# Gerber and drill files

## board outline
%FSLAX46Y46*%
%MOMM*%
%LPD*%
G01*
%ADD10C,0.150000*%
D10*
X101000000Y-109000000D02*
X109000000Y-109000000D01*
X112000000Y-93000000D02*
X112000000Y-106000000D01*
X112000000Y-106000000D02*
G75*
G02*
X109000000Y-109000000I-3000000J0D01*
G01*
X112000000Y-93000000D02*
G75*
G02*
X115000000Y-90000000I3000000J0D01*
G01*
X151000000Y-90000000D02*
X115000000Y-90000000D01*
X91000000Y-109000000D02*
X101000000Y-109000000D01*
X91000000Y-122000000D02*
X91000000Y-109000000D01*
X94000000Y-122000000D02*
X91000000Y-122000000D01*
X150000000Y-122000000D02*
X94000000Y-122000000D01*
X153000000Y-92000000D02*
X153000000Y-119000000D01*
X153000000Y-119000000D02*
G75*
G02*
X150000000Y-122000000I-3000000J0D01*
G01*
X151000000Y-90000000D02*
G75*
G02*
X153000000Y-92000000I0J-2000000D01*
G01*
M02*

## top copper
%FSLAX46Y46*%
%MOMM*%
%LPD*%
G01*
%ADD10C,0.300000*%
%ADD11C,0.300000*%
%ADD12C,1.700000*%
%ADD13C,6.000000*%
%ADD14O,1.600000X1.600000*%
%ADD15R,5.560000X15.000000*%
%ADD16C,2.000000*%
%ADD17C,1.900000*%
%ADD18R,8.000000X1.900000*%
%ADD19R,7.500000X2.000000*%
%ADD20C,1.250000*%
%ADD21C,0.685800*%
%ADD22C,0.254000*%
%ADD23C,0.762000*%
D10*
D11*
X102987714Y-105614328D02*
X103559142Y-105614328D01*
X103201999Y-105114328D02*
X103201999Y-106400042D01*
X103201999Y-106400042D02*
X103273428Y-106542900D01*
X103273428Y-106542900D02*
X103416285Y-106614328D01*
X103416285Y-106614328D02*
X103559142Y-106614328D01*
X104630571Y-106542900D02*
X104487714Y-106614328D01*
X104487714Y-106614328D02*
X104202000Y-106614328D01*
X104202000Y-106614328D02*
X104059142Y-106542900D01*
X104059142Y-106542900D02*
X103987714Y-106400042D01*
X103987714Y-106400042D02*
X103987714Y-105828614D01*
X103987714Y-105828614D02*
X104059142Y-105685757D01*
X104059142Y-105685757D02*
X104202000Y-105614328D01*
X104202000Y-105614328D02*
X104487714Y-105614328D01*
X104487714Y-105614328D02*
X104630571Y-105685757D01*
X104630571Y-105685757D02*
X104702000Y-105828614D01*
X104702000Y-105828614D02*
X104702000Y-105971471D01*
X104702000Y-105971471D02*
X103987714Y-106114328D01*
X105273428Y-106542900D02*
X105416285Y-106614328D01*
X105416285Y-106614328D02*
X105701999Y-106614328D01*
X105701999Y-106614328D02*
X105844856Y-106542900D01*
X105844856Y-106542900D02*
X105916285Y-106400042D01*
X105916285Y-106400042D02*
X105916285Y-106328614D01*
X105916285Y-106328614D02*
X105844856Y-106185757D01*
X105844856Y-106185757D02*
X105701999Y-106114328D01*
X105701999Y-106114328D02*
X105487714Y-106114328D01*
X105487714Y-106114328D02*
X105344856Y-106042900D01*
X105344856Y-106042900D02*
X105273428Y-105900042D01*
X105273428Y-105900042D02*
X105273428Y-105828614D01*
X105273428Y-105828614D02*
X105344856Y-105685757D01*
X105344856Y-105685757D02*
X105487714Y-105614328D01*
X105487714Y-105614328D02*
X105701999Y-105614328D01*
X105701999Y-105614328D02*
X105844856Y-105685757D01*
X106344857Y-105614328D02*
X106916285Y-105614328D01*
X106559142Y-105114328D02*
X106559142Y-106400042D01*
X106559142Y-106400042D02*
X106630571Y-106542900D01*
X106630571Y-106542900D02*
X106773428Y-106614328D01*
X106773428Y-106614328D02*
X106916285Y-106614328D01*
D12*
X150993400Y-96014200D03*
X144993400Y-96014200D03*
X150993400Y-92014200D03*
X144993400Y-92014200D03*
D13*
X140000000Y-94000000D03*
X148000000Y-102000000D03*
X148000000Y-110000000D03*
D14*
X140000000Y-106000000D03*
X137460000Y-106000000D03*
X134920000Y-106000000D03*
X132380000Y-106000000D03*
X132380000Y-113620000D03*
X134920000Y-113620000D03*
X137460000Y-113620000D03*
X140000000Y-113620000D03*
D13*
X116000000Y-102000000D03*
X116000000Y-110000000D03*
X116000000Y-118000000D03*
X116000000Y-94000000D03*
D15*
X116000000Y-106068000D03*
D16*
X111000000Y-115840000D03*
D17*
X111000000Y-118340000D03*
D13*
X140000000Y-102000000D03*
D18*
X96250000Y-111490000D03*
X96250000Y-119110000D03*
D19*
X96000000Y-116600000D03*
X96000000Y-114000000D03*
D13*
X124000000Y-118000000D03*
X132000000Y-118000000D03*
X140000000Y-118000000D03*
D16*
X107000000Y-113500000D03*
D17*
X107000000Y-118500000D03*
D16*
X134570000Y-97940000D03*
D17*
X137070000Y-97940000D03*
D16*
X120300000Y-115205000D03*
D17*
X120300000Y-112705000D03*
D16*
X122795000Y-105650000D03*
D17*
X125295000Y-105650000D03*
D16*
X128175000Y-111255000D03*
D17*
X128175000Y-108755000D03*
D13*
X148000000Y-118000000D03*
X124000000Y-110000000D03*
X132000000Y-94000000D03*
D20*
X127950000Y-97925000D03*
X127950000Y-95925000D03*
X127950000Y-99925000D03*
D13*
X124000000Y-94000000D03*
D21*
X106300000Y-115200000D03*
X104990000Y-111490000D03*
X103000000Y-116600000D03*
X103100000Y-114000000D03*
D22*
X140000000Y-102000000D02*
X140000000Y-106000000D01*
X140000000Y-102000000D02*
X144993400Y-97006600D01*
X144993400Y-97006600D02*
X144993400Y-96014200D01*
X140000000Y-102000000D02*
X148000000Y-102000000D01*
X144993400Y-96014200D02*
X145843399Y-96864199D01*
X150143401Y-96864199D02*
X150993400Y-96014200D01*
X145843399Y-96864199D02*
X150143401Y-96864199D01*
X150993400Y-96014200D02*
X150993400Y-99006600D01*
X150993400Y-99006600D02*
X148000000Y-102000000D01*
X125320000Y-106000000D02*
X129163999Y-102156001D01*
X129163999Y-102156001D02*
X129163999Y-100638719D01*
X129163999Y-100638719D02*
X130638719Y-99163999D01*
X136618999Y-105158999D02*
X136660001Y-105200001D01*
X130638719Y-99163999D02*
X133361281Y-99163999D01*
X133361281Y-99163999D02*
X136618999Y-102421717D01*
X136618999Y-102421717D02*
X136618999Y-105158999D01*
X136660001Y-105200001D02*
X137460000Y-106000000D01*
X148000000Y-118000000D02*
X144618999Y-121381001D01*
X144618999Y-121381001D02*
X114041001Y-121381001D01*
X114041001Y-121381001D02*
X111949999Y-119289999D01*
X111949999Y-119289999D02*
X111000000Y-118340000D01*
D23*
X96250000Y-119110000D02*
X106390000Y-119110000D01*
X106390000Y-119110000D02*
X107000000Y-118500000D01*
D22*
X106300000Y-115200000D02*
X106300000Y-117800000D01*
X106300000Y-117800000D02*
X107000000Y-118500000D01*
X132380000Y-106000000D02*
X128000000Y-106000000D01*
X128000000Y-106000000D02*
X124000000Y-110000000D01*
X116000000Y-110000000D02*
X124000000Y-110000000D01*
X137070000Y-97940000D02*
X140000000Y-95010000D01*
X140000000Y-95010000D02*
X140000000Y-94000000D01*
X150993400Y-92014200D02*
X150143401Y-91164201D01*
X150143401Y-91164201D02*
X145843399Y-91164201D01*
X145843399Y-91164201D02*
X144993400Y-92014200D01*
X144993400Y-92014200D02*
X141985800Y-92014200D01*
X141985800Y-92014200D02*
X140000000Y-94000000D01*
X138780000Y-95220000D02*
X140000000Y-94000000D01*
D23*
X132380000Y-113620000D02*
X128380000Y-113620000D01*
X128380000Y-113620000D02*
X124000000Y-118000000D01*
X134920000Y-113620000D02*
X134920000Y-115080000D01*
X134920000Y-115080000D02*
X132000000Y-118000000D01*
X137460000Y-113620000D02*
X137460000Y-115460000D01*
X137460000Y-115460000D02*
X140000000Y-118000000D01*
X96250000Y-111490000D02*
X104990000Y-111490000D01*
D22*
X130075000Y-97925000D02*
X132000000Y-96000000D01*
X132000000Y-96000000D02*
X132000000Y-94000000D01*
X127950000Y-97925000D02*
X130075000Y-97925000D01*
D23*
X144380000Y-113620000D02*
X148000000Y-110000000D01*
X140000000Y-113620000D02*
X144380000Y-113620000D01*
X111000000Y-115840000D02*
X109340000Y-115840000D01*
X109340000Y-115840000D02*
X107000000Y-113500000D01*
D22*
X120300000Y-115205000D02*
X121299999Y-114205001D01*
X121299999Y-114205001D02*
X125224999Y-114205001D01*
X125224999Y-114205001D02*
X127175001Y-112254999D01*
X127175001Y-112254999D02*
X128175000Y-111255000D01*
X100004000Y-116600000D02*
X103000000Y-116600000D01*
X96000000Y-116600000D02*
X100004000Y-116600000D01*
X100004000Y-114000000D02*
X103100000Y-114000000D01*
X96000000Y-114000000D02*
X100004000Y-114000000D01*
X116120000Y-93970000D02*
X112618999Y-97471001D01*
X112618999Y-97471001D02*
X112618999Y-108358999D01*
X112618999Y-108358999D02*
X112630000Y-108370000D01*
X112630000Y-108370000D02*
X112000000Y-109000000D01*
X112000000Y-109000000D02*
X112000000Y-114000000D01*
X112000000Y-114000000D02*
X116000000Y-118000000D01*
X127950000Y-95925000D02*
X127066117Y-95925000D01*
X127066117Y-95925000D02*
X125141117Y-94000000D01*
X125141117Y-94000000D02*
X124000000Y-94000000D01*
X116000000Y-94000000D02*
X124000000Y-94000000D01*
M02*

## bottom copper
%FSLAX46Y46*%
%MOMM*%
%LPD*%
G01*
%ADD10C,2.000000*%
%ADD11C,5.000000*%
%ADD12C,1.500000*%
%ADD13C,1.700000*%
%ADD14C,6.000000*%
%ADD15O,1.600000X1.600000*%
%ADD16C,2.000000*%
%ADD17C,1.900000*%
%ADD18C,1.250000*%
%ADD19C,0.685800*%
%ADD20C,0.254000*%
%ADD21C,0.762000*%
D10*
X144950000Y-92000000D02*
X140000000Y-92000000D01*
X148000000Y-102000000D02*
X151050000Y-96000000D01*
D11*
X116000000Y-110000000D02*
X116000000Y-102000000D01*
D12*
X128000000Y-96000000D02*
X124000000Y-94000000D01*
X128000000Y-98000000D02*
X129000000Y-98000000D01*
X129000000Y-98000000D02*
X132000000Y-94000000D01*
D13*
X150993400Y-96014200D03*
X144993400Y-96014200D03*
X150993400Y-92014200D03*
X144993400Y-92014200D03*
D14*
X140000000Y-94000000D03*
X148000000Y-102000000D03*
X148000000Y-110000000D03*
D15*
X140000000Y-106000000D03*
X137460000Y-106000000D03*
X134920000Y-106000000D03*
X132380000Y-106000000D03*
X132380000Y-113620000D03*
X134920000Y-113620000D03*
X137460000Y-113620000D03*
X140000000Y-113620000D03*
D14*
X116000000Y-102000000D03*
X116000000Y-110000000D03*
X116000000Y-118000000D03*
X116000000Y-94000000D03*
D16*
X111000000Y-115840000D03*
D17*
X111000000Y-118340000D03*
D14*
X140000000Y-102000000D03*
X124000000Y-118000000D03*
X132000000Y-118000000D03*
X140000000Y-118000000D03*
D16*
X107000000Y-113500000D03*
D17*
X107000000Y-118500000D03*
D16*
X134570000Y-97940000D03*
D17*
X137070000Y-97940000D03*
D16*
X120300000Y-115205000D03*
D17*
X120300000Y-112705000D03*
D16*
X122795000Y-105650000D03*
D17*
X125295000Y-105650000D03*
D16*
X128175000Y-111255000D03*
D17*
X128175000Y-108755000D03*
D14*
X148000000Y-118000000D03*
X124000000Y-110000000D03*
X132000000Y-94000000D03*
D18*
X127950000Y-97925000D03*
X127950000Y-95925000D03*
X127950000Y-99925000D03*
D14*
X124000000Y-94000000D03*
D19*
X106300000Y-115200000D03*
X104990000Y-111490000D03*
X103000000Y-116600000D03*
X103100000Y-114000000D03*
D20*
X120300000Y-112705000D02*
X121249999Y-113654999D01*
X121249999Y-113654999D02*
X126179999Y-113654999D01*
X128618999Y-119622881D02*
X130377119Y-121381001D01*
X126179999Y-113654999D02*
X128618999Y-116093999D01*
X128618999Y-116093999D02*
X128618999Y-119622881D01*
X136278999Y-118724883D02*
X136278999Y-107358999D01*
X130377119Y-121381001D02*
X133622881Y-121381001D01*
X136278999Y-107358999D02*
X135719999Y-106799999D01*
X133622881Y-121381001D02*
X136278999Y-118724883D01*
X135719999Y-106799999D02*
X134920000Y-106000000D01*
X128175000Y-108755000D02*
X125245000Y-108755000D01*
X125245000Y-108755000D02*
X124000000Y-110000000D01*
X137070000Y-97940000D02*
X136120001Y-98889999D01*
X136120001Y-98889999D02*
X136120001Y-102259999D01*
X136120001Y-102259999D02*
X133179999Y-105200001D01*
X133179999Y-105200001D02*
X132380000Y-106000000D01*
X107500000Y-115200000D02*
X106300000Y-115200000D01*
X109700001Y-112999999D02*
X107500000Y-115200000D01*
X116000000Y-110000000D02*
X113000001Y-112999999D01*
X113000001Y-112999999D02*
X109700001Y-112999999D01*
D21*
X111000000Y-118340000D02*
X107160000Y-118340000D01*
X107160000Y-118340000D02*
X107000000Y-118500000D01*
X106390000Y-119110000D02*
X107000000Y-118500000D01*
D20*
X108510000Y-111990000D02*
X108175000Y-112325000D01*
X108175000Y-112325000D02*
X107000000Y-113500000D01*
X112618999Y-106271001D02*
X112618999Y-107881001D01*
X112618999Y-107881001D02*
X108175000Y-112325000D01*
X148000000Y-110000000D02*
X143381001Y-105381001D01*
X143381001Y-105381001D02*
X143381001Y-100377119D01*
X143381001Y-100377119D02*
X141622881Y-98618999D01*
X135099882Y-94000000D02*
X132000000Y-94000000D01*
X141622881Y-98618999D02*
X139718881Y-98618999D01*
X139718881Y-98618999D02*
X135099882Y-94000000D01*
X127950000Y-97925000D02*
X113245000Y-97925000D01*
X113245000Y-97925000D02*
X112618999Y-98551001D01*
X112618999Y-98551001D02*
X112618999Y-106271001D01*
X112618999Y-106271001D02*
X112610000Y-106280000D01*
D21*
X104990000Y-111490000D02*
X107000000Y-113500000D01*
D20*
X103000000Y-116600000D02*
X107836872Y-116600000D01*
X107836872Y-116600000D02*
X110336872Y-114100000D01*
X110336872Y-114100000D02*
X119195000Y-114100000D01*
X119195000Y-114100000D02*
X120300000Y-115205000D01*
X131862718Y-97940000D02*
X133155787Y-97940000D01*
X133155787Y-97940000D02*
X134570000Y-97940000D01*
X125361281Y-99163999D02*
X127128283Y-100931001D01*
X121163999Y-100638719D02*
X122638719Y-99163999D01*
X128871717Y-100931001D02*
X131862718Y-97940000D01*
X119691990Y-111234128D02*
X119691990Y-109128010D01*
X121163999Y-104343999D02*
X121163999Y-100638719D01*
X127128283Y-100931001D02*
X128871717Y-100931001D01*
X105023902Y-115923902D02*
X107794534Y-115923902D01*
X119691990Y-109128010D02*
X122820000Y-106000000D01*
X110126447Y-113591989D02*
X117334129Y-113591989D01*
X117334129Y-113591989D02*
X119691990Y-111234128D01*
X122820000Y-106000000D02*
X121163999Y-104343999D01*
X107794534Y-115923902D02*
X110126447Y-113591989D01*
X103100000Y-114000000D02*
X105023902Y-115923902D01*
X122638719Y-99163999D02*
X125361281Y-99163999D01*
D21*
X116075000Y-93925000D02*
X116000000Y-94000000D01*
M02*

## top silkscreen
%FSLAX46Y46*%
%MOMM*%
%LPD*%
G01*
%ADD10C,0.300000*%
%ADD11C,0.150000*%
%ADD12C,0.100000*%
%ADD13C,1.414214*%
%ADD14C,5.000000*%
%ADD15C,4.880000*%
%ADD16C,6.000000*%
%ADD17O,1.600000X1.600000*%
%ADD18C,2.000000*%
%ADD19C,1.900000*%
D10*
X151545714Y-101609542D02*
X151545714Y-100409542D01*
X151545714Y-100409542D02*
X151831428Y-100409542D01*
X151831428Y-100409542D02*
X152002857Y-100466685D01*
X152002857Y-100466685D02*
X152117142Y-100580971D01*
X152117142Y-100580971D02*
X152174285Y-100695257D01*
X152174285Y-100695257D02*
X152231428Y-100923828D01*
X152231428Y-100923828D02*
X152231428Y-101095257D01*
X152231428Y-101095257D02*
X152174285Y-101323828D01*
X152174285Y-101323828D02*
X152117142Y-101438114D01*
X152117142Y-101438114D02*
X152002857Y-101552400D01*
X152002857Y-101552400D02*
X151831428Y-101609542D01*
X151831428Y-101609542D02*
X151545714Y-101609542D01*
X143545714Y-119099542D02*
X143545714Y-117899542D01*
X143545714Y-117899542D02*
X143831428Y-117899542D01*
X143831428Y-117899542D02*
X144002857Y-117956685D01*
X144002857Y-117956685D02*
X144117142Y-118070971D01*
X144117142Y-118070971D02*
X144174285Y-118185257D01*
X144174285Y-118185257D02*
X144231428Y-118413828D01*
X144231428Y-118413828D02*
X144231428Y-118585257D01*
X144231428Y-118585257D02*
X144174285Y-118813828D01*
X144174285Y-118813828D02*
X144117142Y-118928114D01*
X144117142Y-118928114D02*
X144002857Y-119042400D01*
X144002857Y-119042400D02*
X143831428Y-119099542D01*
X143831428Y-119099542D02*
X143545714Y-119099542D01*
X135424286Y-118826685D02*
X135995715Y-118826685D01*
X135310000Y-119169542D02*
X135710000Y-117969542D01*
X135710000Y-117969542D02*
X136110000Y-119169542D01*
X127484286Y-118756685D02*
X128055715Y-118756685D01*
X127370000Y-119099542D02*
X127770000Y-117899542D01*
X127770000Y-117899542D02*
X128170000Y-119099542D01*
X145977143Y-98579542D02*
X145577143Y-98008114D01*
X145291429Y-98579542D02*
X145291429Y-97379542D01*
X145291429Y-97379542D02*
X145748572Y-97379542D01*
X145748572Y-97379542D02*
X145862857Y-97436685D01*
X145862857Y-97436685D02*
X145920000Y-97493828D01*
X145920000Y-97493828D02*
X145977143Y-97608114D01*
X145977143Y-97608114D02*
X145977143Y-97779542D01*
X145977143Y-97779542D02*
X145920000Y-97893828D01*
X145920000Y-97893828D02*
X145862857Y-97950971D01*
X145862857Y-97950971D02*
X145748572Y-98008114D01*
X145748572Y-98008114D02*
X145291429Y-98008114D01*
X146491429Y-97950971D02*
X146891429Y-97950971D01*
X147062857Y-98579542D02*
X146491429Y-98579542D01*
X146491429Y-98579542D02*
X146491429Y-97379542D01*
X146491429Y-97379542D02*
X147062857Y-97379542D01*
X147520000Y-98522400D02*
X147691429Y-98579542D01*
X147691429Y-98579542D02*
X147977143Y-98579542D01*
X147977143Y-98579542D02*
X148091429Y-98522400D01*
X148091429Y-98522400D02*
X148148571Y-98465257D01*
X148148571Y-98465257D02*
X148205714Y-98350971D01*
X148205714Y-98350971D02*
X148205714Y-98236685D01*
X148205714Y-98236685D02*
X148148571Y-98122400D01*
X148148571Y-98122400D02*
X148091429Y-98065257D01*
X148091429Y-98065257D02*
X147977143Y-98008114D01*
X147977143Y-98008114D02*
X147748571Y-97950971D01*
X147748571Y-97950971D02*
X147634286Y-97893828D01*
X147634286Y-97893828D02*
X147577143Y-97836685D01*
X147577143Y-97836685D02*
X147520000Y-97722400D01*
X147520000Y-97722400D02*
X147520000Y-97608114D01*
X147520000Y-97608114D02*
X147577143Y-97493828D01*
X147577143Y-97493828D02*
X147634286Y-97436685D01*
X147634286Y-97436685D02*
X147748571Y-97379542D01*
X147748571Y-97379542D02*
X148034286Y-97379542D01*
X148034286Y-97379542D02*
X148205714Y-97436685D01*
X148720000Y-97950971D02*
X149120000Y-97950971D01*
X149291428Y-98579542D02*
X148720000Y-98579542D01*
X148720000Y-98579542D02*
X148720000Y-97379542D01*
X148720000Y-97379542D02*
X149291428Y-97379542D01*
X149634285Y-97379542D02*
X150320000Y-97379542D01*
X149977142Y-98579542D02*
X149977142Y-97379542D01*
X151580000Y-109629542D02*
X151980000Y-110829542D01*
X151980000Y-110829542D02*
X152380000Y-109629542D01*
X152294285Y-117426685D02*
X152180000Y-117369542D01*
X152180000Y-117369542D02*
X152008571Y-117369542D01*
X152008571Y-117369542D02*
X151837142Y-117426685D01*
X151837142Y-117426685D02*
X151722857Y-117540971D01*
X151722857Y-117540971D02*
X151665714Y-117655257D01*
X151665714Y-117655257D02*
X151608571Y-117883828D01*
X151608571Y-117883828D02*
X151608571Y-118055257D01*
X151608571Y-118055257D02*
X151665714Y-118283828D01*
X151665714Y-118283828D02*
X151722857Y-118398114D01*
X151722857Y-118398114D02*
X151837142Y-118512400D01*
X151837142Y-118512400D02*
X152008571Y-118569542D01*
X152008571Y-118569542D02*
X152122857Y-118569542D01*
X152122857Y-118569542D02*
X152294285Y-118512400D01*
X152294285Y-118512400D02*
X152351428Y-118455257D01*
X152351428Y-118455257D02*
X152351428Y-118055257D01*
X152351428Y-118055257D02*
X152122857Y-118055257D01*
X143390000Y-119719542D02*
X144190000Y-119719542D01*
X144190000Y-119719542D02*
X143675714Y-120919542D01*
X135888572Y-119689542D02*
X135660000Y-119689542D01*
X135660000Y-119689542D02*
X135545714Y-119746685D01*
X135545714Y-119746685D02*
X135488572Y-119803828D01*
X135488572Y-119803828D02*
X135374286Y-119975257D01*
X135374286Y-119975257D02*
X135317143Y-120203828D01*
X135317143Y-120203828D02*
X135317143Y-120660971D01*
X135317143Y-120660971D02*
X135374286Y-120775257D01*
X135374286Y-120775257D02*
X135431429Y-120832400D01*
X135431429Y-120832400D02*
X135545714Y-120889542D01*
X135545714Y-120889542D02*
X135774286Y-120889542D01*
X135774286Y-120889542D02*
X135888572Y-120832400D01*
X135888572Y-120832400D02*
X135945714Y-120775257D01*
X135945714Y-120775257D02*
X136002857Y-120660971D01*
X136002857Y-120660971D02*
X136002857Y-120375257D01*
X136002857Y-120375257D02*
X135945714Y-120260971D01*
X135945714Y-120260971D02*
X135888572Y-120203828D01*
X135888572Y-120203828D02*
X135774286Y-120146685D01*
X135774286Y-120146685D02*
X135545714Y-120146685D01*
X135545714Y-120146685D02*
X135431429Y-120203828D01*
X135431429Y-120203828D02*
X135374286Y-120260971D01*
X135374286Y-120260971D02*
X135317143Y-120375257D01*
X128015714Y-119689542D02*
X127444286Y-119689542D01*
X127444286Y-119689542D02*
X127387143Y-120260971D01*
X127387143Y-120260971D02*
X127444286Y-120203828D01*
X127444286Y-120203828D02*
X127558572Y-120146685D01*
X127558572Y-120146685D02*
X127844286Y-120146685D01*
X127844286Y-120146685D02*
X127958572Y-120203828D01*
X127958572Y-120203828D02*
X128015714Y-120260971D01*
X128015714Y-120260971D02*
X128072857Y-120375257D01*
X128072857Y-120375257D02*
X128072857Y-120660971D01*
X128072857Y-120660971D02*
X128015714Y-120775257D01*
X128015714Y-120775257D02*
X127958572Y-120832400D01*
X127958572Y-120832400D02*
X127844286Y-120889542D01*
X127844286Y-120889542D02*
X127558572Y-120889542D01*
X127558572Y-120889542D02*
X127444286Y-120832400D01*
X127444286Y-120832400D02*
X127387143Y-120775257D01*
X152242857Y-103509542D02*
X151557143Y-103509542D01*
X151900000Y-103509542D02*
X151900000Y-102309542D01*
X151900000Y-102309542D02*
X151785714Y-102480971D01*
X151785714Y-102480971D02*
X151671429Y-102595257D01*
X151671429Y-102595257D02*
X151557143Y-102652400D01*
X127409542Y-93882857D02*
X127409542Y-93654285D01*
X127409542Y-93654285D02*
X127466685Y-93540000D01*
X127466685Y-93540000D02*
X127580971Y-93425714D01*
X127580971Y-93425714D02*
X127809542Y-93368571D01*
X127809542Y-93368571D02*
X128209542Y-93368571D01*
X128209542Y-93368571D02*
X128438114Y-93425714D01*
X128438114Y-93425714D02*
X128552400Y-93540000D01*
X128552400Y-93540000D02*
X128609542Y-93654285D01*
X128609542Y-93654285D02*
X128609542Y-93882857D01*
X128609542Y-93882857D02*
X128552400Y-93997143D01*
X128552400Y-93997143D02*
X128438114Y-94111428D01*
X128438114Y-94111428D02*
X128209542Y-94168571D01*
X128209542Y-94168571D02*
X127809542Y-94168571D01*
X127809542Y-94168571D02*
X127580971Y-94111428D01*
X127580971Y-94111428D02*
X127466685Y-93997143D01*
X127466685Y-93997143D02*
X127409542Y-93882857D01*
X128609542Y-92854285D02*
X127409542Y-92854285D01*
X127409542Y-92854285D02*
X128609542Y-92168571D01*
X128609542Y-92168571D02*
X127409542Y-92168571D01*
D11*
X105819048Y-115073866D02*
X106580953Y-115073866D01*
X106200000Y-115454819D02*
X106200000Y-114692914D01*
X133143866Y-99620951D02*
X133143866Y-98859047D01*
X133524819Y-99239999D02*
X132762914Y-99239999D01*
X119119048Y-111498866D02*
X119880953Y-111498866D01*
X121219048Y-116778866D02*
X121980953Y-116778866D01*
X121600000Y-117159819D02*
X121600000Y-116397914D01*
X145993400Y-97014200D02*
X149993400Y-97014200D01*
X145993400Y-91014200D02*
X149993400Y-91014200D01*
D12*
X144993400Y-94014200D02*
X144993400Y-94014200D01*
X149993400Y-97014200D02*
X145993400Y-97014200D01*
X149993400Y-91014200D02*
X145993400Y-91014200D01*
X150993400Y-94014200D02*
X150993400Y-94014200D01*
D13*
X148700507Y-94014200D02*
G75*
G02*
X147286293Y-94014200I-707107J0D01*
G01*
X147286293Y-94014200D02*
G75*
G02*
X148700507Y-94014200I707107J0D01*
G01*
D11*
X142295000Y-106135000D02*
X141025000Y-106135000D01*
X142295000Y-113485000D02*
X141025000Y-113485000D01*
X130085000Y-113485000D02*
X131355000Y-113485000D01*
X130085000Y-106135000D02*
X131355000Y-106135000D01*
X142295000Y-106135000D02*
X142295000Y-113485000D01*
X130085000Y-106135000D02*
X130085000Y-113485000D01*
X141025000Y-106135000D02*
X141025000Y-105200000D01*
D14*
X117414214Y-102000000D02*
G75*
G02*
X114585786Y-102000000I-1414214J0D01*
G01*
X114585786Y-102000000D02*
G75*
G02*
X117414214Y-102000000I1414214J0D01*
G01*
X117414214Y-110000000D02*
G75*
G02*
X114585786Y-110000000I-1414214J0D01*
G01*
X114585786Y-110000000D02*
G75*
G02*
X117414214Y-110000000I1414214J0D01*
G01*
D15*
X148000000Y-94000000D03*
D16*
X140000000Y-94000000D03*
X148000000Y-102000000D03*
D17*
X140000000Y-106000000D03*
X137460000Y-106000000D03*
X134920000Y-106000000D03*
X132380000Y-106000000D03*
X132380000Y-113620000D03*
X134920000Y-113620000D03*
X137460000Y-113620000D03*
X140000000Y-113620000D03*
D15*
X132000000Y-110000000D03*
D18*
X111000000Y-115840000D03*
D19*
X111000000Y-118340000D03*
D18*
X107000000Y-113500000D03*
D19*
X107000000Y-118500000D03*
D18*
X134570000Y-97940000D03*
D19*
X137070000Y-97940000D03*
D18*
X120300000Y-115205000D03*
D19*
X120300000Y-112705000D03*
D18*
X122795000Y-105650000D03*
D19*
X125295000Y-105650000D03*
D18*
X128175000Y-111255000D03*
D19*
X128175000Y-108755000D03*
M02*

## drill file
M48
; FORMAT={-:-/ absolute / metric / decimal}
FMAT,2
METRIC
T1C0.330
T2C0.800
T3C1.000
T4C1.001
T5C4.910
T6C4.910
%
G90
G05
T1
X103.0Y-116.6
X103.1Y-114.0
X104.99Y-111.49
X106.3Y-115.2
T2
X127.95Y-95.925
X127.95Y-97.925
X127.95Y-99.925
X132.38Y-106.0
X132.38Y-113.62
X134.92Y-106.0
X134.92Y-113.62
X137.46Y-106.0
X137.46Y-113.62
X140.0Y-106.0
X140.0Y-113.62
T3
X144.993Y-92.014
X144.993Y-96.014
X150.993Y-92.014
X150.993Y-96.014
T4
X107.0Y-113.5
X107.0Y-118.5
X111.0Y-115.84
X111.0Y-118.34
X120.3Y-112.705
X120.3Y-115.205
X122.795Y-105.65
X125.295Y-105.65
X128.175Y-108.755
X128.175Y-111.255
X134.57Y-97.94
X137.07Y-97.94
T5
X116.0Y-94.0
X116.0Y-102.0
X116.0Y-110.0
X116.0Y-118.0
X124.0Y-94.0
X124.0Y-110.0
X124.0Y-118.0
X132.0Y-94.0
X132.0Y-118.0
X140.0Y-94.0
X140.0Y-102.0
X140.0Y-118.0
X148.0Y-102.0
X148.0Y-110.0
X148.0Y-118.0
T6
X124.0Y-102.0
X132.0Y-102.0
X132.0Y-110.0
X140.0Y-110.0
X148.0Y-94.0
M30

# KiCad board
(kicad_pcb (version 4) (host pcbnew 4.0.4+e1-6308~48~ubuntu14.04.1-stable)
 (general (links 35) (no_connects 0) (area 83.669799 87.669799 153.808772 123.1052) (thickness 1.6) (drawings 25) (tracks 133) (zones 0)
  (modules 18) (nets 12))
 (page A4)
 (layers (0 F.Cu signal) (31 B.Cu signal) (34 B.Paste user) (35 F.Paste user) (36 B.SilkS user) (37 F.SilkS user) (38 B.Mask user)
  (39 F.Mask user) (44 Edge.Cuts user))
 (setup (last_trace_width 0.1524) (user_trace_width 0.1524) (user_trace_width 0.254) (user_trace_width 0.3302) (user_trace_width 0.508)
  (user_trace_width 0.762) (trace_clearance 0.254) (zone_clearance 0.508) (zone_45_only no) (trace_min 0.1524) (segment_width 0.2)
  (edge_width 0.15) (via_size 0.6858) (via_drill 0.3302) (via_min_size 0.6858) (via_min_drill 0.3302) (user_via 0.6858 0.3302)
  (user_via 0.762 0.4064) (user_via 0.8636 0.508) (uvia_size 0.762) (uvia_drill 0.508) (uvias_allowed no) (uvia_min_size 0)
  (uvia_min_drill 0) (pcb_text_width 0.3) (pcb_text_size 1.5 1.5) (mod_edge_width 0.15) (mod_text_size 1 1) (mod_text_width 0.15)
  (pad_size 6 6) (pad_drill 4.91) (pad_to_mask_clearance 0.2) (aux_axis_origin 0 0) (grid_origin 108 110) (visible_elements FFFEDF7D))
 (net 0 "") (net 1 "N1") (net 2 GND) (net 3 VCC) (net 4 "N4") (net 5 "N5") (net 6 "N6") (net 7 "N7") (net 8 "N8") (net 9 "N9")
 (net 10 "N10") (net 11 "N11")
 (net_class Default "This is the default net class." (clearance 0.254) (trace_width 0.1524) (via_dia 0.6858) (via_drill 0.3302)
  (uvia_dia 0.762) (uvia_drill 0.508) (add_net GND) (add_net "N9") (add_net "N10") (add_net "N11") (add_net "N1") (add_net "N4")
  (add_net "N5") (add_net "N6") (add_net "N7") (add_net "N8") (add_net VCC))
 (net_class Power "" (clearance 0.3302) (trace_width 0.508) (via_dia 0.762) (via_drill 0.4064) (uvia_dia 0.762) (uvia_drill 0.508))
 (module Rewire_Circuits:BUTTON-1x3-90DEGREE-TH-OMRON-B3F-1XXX (layer F.Cu) (at 148 94)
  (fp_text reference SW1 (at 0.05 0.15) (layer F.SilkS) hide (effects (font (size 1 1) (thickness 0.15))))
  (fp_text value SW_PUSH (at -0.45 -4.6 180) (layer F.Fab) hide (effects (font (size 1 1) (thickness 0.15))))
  (fp_line (start -3.05 -2) (end -8 -2) (layer B.Cu) (width 2))
  (fp_line (start -2.0066 3.0142) (end 1.9934 3.0142) (layer F.SilkS) (width 0.15))
  (fp_line (start -2.0066 -2.9858) (end 1.9934 -2.9858) (layer F.SilkS) (width 0.15))
  (fp_line (start -3.0066 0.0142) (end -3.0066 0.0142) (layer F.SilkS) (width 0))
  (fp_line (start 1.9934 3.0142) (end -2.0066 3.0142) (layer F.SilkS) (width 0))
  (fp_line (start 1.9934 -2.9858) (end -2.0066 -2.9858) (layer F.SilkS) (width 0))
  (fp_line (start 2.9934 0.0142) (end 2.9934 0.0142) (layer F.SilkS) (width 0))
  (fp_circle (center -0.0066 0.0142) (end 0.9934 1.0142) (layer F.SilkS) (width 0))
  (fp_line (start 0 8) (end 3.05 2) (layer B.Cu) (width 2))
  (pad 2 thru_hole circle (at 2.9934 2.0142) (size 1.7 1.7) (drill 1) (layers *.Cu *.Mask) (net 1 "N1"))
  (pad 2 thru_hole circle (at -3.0066 2.0142) (size 1.7 1.7) (drill 1) (layers *.Cu *.Mask) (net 1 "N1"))
  (pad 1 thru_hole circle (at 2.9934 -1.9858) (size 1.7 1.7) (drill 1) (layers *.Cu *.Mask) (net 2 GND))
  (pad 1 thru_hole circle (at -3.0066 -1.9858) (size 1.7 1.7) (drill 1) (layers *.Cu *.Mask) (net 2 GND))
  (pad "" np_thru_hole circle (at 0 0) (size 4.88 4.88) (drill 4.91) (layers *.Cu *.Mask F.SilkS))
  (pad 1 thru_hole circle (at -8 0) (size 6 6) (drill 4.91) (layers *.Cu *.Mask F.SilkS) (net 2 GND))
  (pad 2 thru_hole circle (at 0 8) (size 6 6) (drill 4.91) (layers *.Cu *.Mask F.SilkS) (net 1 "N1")))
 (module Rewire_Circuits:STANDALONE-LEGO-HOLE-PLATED (layer F.Cu) (at 148 110)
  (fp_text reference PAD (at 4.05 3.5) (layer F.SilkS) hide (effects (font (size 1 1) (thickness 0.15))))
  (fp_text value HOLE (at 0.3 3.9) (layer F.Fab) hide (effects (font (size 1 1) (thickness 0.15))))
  (pad 1 thru_hole circle (at 0 0) (size 6 6) (drill 4.91) (layers *.Cu *.Mask) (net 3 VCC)))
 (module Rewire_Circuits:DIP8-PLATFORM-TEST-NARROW (layer F.Cu) (at 136 110 180)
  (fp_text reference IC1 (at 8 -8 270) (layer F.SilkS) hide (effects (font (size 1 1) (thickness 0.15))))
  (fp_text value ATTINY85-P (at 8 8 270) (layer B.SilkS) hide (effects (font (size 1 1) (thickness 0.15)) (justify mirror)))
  (fp_line (start -6.295 3.865) (end -5.025 3.865) (layer F.SilkS) (width 0.15))
  (fp_line (start -6.295 -3.485) (end -5.025 -3.485) (layer F.SilkS) (width 0.15))
  (fp_line (start 5.915 -3.485) (end 4.645 -3.485) (layer F.SilkS) (width 0.15))
  (fp_line (start 5.915 3.865) (end 4.645 3.865) (layer F.SilkS) (width 0.15))
  (fp_line (start -6.295 3.865) (end -6.295 -3.485) (layer F.SilkS) (width 0.15))
  (fp_line (start 5.915 3.865) (end 5.915 -3.485) (layer F.SilkS) (width 0.15))
  (fp_line (start -5.025 3.865) (end -5.025 4.8) (layer F.SilkS) (width 0.15))
  (pad 1 thru_hole oval (at -4 4 270) (size 1.6 1.6) (drill 0.8) (layers *.Cu *.Mask F.SilkS) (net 1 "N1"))
  (pad 2 thru_hole oval (at -1.46 4 270) (size 1.6 1.6) (drill 0.8) (layers *.Cu *.Mask F.SilkS) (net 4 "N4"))
  (pad 3 thru_hole oval (at 1.08 4 270) (size 1.6 1.6) (drill 0.8) (layers *.Cu *.Mask F.SilkS) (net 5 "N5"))
  (pad 4 thru_hole oval (at 3.62 4 270) (size 1.6 1.6) (drill 0.8) (layers *.Cu *.Mask F.SilkS) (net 2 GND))
  (pad 5 thru_hole oval (at 3.62 -3.62 270) (size 1.6 1.6) (drill 0.8) (layers *.Cu *.Mask F.SilkS) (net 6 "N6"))
  (pad 6 thru_hole oval (at 1.08 -3.62 270) (size 1.6 1.6) (drill 0.8) (layers *.Cu *.Mask F.SilkS) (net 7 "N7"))
  (pad 7 thru_hole oval (at -1.46 -3.62 270) (size 1.6 1.6) (drill 0.8) (layers *.Cu *.Mask F.SilkS) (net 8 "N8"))
  (pad 8 thru_hole oval (at -4 -3.62 270) (size 1.6 1.6) (drill 0.8) (layers *.Cu *.Mask F.SilkS) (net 3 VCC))
  (pad "" np_thru_hole circle (at -4 0 180) (size 4.88 4.88) (drill 4.91) (layers *.Cu *.Mask))
  (pad "" np_thru_hole circle (at 4 0 180) (size 4.88 4.88) (drill 4.91) (layers *.Cu *.Mask F.SilkS)))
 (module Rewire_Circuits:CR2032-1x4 (layer F.Cu) (at 116 106 90)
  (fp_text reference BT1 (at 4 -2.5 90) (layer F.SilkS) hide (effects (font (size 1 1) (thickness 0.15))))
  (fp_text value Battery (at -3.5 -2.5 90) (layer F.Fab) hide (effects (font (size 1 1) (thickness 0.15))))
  (fp_circle (center 4 0) (end 5 1) (layer F.SilkS) (width 5))
  (fp_circle (center -4 0) (end -3 1) (layer F.SilkS) (width 5)) (fp_line (start -4 0) (end 4 0) (layer B.Cu) (width 5))
  (pad GND thru_hole circle (at 4 0 90) (size 6 6) (drill 4.91) (layers *.Cu *.Mask) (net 2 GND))
  (pad GND thru_hole circle (at -4 0 90) (size 6 6) (drill 4.91) (layers *.Cu *.Mask) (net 2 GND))
  (pad 1 thru_hole circle (at -12 0 90) (size 6 6) (drill 4.91) (layers *.Cu *.Mask) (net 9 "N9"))
  (pad 1 thru_hole circle (at 12 0 90) (size 6 6) (drill 4.91) (layers *.Cu *.Mask) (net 9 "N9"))
  (pad GND smd rect (at -0.068 0 90) (size 15 5.56) (layers F.Cu F.Paste F.Mask) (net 2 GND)))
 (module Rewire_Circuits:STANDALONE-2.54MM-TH (layer F.Cu) (at 111 117.12)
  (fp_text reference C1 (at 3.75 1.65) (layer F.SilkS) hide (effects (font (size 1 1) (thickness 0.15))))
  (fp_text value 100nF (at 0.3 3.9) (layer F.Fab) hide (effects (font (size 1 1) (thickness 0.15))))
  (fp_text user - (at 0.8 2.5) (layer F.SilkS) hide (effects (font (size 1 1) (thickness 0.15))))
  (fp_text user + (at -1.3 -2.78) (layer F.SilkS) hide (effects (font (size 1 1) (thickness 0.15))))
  (pad 1 thru_hole circle (at 0 -1.28) (size 2 2) (drill 1.00076) (layers *.Cu *.Mask F.SilkS) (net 3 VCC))
  (pad 2 thru_hole circle (at 0 1.22 270) (size 1.9 1.9) (drill 1.00076) (layers *.Cu *.Mask F.SilkS) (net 2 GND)))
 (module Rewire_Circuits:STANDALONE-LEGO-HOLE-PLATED (layer F.Cu) (at 140 102 180)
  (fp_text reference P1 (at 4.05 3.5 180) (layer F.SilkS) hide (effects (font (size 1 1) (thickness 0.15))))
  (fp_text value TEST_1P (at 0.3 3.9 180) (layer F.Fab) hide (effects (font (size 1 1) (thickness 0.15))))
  (pad 1 thru_hole circle (at 0 0 180) (size 6 6) (drill 4.91) (layers *.Cu *.Mask) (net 1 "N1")))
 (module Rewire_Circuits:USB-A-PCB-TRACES (layer F.Cu) (at 101.15 115.3 90)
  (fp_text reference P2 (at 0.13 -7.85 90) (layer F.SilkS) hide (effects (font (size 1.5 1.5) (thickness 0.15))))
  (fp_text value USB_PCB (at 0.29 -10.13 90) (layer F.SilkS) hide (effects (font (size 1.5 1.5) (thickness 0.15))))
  (pad 1 connect rect (at 3.81 -4.9 90) (size 1.9 8) (layers F.Cu F.Mask) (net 3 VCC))
  (pad 4 connect rect (at -3.81 -4.9 90) (size 1.9 8) (layers F.Cu F.Mask) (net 2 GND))
  (pad 3 connect rect (at -1.3 -5.15 90) (size 2 7.5) (layers F.Cu F.Mask) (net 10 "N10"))
  (pad 2 connect rect (at 1.3 -5.15 90) (size 2 7.5) (layers F.Cu F.Mask) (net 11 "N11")))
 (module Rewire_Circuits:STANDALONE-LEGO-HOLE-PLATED (layer F.Cu) (at 124 118 180)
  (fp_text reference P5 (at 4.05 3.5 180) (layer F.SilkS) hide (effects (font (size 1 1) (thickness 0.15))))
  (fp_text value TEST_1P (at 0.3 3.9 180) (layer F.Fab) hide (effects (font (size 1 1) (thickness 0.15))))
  (pad 1 thru_hole circle (at 0 0 180) (size 6 6) (drill 4.91) (layers *.Cu *.Mask) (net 6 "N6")))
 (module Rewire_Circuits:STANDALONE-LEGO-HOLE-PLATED (layer F.Cu) (at 132 118 180)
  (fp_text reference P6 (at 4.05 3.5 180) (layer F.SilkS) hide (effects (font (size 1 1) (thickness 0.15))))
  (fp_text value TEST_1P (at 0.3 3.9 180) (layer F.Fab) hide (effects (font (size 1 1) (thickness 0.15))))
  (pad 1 thru_hole circle (at 0 0 180) (size 6 6) (drill 4.91) (layers *.Cu *.Mask) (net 7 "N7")))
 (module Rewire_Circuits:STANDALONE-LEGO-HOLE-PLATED (layer F.Cu) (at 140 118 180)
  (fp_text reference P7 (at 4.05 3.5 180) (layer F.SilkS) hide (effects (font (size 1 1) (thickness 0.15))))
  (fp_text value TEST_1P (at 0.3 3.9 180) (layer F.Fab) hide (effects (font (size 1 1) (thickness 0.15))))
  (pad 1 thru_hole circle (at 0 0 180) (size 6 6) (drill 4.91) (layers *.Cu *.Mask) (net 8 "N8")))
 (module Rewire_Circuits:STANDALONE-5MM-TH (layer F.Cu) (at 107 116)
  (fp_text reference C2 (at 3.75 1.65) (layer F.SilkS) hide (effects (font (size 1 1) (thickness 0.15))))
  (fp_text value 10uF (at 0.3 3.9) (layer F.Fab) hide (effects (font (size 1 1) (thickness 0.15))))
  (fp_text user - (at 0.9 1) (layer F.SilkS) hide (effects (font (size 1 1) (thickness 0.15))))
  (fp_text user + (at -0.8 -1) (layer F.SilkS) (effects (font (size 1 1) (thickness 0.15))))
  (pad 1 thru_hole circle (at 0 -2.5) (size 2 2) (drill 1.00076) (layers *.Cu *.Mask F.SilkS) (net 3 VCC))
  (pad 2 thru_hole circle (at 0 2.5 270) (size 1.9 1.9) (drill 1.00076) (layers *.Cu *.Mask F.SilkS) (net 2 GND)))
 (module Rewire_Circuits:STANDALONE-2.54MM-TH (layer F.Cu) (at 135.85 97.94 90)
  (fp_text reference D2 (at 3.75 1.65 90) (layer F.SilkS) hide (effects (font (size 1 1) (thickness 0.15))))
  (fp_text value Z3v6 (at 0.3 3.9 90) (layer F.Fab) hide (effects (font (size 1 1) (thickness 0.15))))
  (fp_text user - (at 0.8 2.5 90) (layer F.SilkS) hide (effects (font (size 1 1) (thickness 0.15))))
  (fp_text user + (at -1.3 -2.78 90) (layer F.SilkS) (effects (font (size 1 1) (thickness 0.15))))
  (pad 1 thru_hole circle (at 0 -1.28 90) (size 2 2) (drill 1.00076) (layers *.Cu *.Mask F.SilkS) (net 11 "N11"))
  (pad 2 thru_hole circle (at 0 1.22) (size 1.9 1.9) (drill 1.00076) (layers *.Cu *.Mask F.SilkS) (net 2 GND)))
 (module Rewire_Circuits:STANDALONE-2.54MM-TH (layer F.Cu) (at 120.3 113.925 180)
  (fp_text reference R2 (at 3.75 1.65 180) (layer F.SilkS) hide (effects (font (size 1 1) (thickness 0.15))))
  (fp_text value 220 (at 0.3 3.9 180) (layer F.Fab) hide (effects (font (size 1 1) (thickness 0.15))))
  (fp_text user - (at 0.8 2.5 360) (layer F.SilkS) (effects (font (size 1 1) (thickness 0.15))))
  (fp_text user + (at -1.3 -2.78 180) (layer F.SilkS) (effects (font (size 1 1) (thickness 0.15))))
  (pad 1 thru_hole circle (at 0 -1.28 180) (size 2 2) (drill 1.00076) (layers *.Cu *.Mask F.SilkS) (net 10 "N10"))
  (pad 2 thru_hole circle (at 0 1.22 90) (size 1.9 1.9) (drill 1.00076) (layers *.Cu *.Mask F.SilkS) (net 5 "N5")))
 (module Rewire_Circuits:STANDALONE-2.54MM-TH (layer F.Cu) (at 124.075 105.65 90)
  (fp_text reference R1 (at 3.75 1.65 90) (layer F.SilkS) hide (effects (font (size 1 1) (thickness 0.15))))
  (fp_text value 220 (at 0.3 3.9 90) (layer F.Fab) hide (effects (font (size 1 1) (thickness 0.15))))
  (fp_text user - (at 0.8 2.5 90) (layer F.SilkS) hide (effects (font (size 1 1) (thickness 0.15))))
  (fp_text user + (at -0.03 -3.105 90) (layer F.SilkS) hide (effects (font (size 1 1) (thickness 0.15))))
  (pad 1 thru_hole circle (at 0 -1.28 90) (size 2 2) (drill 1.00076) (layers *.Cu *.Mask F.SilkS) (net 11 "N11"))
  (pad 2 thru_hole circle (at 0 1.22) (size 1.9 1.9) (drill 1.00076) (layers *.Cu *.Mask F.SilkS) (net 4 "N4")))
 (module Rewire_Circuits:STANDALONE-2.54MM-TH (layer F.Cu) (at 128.175 109.975 180)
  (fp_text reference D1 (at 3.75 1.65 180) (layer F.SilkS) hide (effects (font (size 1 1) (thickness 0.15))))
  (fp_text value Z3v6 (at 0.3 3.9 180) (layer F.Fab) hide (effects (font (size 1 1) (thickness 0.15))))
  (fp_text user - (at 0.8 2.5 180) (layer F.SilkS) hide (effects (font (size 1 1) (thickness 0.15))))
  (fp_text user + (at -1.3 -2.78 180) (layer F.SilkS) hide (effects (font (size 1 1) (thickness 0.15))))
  (pad 1 thru_hole circle (at 0 -1.28 180) (size 2 2) (drill 1.00076) (layers *.Cu *.Mask F.SilkS) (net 10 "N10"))
  (pad 2 thru_hole circle (at 0 1.22 90) (size 1.9 1.9) (drill 1.00076) (layers *.Cu *.Mask F.SilkS) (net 2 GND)))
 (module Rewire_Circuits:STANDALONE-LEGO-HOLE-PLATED (layer F.Cu) (at 148 118)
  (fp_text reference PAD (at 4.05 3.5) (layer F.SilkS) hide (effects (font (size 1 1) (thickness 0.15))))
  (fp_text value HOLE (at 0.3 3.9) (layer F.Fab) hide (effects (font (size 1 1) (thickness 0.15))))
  (pad 1 thru_hole circle (at 0 0) (size 6 6) (drill 4.91) (layers *.Cu *.Mask) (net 2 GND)))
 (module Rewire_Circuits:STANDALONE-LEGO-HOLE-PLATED (layer F.Cu) (at 124 110)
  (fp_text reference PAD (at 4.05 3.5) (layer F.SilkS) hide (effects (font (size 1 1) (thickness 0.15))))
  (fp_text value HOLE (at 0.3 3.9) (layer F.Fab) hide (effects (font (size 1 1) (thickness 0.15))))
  (pad 1 thru_hole circle (at 0 0) (size 6 6) (drill 4.91) (layers *.Cu *.Mask) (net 2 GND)))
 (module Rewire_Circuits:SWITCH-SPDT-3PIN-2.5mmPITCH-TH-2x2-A (layer F.Cu) (at 128 102)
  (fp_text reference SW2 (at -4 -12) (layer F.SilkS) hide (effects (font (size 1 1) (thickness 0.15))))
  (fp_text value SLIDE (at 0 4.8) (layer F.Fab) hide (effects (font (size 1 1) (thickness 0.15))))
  (fp_line (start 0 -6) (end -4 -8) (layer B.Cu) (width 1.5)) (fp_line (start 0 -4) (end 1 -4) (layer B.Cu) (width 1.5))
  (fp_line (start 1 -4) (end 4 -8) (layer B.Cu) (width 1.5))
  (pad 2 thru_hole circle (at 4 -8) (size 6 6) (drill 4.91) (layers *.Cu *.Mask) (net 3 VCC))
  (pad 2 thru_hole circle (at -0.05 -4.075 270) (size 1.25 1.25) (drill 0.8) (layers *.Cu *.Mask) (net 3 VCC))
  (pad 3 thru_hole circle (at -0.05 -6.075 270) (size 1.25 1.25) (drill 0.8) (layers *.Cu *.Mask) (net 9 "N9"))
  (pad 1 thru_hole circle (at -0.05 -2.075 270) (size 1.25 1.25) (drill 0.8) (layers *.Cu *.Mask))
  (pad "" np_thru_hole circle (at 4 0) (size 4.91 4.91) (drill 4.91) (layers *.Cu))
  (pad 3 thru_hole circle (at -4 -8) (size 6 6) (drill 4.91) (layers *.Cu *.Mask) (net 9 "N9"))
  (pad "" np_thru_hole circle (at -4 0) (size 4.91 4.91) (drill 4.91) (layers *.Cu)))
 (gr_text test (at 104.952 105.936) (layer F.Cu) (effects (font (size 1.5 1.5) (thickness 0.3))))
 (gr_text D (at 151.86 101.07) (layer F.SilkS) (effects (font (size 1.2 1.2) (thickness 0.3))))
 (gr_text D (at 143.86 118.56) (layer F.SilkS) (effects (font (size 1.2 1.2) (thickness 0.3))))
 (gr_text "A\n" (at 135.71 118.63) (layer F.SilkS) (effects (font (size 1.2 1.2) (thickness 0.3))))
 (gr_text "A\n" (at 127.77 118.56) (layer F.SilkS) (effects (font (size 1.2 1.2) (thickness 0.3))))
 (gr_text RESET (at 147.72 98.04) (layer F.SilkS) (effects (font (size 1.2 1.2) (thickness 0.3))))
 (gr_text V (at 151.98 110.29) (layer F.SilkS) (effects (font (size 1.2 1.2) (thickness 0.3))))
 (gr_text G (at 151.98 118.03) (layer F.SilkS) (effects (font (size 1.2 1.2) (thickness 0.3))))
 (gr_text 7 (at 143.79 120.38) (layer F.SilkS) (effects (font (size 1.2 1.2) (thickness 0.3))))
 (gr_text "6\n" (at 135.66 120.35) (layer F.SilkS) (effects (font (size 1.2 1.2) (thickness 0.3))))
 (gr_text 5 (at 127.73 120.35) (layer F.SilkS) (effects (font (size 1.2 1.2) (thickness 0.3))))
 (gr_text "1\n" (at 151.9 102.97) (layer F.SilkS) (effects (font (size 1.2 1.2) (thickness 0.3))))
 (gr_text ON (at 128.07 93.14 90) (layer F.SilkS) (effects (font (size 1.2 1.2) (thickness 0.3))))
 (gr_line (start 101 109) (end 109 109) (layer Edge.Cuts) (width 0.15))
 (gr_line (start 112 93) (end 112 106) (layer Edge.Cuts) (width 0.15))
 (gr_arc (start 109 106) (end 112 106) (angle 90) (layer Edge.Cuts) (width 0.15))
 (gr_arc (start 115 93) (end 112 93) (angle 90) (layer Edge.Cuts) (width 0.15))
 (gr_line (start 151 90) (end 115 90) (layer Edge.Cuts) (width 0.15))
 (gr_line (start 91 109) (end 101 109) (layer Edge.Cuts) (width 0.15))
 (gr_line (start 91 122) (end 91 109) (layer Edge.Cuts) (width 0.15))
 (gr_line (start 94 122) (end 91 122) (layer Edge.Cuts) (width 0.15))
 (gr_line (start 150 122) (end 94 122) (layer Edge.Cuts) (width 0.15))
 (gr_line (start 153 92) (end 153 119) (layer Edge.Cuts) (width 0.15))
 (gr_arc (start 150 119) (end 153 119) (angle 90) (layer Edge.Cuts) (width 0.15))
 (gr_arc (start 151 92) (end 151 90) (angle 90) (layer Edge.Cuts) (width 0.15))
 (segment (start 84 112) (end 84 110) (width 0.1524) (layer Dwgs.User) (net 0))
 (segment (start 84 96) (end 84 88) (width 0.1524) (layer Dwgs.User) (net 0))
 (segment (start 140 102) (end 140 106) (width 0.254) (layer F.Cu) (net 1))
 (segment (start 140 102) (end 144.9934 97.0066) (width 0.254) (layer F.Cu) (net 1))
 (segment (start 144.9934 97.0066) (end 144.9934 96.0142) (width 0.254) (layer F.Cu) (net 1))
 (segment (start 140 102) (end 148 102) (width 0.254) (layer F.Cu) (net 1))
 (segment (start 144.9934 96.0142) (end 145.843399 96.864199) (width 0.254) (layer F.Cu) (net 1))
 (segment (start 150.143401 96.864199) (end 150.9934 96.0142) (width 0.254) (layer F.Cu) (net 1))
 (segment (start 145.843399 96.864199) (end 150.143401 96.864199) (width 0.254) (layer F.Cu) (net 1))
 (segment (start 150.9934 96.0142) (end 150.9934 99.0066) (width 0.254) (layer F.Cu) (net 1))
 (segment (start 150.9934 99.0066) (end 148 102) (width 0.254) (layer F.Cu) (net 1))
 (segment (start 125.32 106) (end 129.163999 102.156001) (width 0.254) (layer F.Cu) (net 4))
 (segment (start 129.163999 102.156001) (end 129.163999 100.638719) (width 0.254) (layer F.Cu) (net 4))
 (segment (start 129.163999 100.638719) (end 130.638719 99.163999) (width 0.254) (layer F.Cu) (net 4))
 (segment (start 136.618999 105.158999) (end 136.660001 105.200001) (width 0.254) (layer F.Cu) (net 4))
 (segment (start 130.638719 99.163999) (end 133.361281 99.163999) (width 0.254) (layer F.Cu) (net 4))
 (segment (start 133.361281 99.163999) (end 136.618999 102.421717) (width 0.254) (layer F.Cu) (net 4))
 (segment (start 136.618999 102.421717) (end 136.618999 105.158999) (width 0.254) (layer F.Cu) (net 4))
 (segment (start 136.660001 105.200001) (end 137.46 106) (width 0.254) (layer F.Cu) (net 4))
 (segment (start 120.3 112.705) (end 121.249999 113.654999) (width 0.254) (layer B.Cu) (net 5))
 (segment (start 121.249999 113.654999) (end 126.179999 113.654999) (width 0.254) (layer B.Cu) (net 5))
 (segment (start 128.618999 119.622881) (end 130.377119 121.381001) (width 0.254) (layer B.Cu) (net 5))
 (segment (start 126.179999 113.654999) (end 128.618999 116.093999) (width 0.254) (layer B.Cu) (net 5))
 (segment (start 128.618999 116.093999) (end 128.618999 119.622881) (width 0.254) (layer B.Cu) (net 5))
 (segment (start 136.278999 118.724883) (end 136.278999 107.358999) (width 0.254) (layer B.Cu) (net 5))
 (segment (start 130.377119 121.381001) (end 133.622881 121.381001) (width 0.254) (layer B.Cu) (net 5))
 (segment (start 136.278999 107.358999) (end 135.719999 106.799999) (width 0.254) (layer B.Cu) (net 5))
 (segment (start 133.622881 121.381001) (end 136.278999 118.724883) (width 0.254) (layer B.Cu) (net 5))
 (segment (start 135.719999 106.799999) (end 134.92 106) (width 0.254) (layer B.Cu) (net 5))
 (segment (start 148 118) (end 144.618999 121.381001) (width 0.254) (layer F.Cu) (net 2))
 (segment (start 144.618999 121.381001) (end 114.041001 121.381001) (width 0.254) (layer F.Cu) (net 2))
 (segment (start 114.041001 121.381001) (end 111.949999 119.289999) (width 0.254) (layer F.Cu) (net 2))
 (segment (start 111.949999 119.289999) (end 111 118.34) (width 0.254) (layer F.Cu) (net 2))
 (segment (start 128.175 108.755) (end 125.245 108.755) (width 0.254) (layer B.Cu) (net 2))
 (segment (start 125.245 108.755) (end 124 110) (width 0.254) (layer B.Cu) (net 2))
 (segment (start 96.25 119.11) (end 106.39 119.11) (width 0.762) (layer F.Cu) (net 2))
 (segment (start 106.39 119.11) (end 107 118.5) (width 0.762) (layer F.Cu) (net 2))
 (segment (start 137.07 97.94) (end 136.120001 98.889999) (width 0.254) (layer B.Cu) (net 2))
 (segment (start 136.120001 98.889999) (end 136.120001 102.259999) (width 0.254) (layer B.Cu) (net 2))
 (segment (start 136.120001 102.259999) (end 133.179999 105.200001) (width 0.254) (layer B.Cu) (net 2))
 (segment (start 133.179999 105.200001) (end 132.38 106) (width 0.254) (layer B.Cu) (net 2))
 (segment (start 106.3 115.2) (end 106.3 117.8) (width 0.254) (layer F.Cu) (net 2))
 (segment (start 106.3 117.8) (end 107 118.5) (width 0.254) (layer F.Cu) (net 2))
 (segment (start 107.5 115.2) (end 106.3 115.2) (width 0.254) (layer B.Cu) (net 2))
 (via (at 106.3 115.2) (size 0.6858) (drill 0.3302) (layers F.Cu B.Cu) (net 2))
 (segment (start 109.700001 112.999999) (end 107.5 115.2) (width 0.254) (layer B.Cu) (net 2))
 (segment (start 116 110) (end 113.000001 112.999999) (width 0.254) (layer B.Cu) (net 2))
 (segment (start 113.000001 112.999999) (end 109.700001 112.999999) (width 0.254) (layer B.Cu) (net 2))
 (segment (start 132.38 106) (end 128 106) (width 0.254) (layer F.Cu) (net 2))
 (segment (start 128 106) (end 124 110) (width 0.254) (layer F.Cu) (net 2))
 (segment (start 116 110) (end 124 110) (width 0.254) (layer F.Cu) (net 2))
 (segment (start 137.07 97.94) (end 140 95.01) (width 0.254) (layer F.Cu) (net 2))
 (segment (start 140 95.01) (end 140 94) (width 0.254) (layer F.Cu) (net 2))
 (segment (start 150.9934 92.0142) (end 150.143401 91.164201) (width 0.254) (layer F.Cu) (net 2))
 (segment (start 150.143401 91.164201) (end 145.843399 91.164201) (width 0.254) (layer F.Cu) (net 2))
 (segment (start 145.843399 91.164201) (end 144.9934 92.0142) (width 0.254) (layer F.Cu) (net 2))
 (segment (start 144.9934 92.0142) (end 141.9858 92.0142) (width 0.254) (layer F.Cu) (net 2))
 (segment (start 141.9858 92.0142) (end 140 94) (width 0.254) (layer F.Cu) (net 2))
 (segment (start 138.78 95.22) (end 140 94) (width 0.254) (layer F.Cu) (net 2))
 (segment (start 111 118.34) (end 107.16 118.34) (width 0.762) (layer B.Cu) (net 2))
 (segment (start 107.16 118.34) (end 107 118.5) (width 0.762) (layer B.Cu) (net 2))
 (segment (start 106.39 119.11) (end 107 118.5) (width 0.762) (layer B.Cu) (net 2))
 (segment (start 132.38 113.62) (end 128.38 113.62) (width 0.762) (layer F.Cu) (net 6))
 (segment (start 128.38 113.62) (end 124 118) (width 0.762) (layer F.Cu) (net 6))
 (segment (start 134.92 113.62) (end 134.92 115.08) (width 0.762) (layer F.Cu) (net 7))
 (segment (start 134.92 115.08) (end 132 118) (width 0.762) (layer F.Cu) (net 7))
 (segment (start 137.46 113.62) (end 137.46 115.46) (width 0.762) (layer F.Cu) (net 8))
 (segment (start 137.46 115.46) (end 140 118) (width 0.762) (layer F.Cu) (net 8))
 (segment (start 108.51 111.99) (end 108.175 112.325) (width 0.254) (layer B.Cu) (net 3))
 (segment (start 108.175 112.325) (end 107 113.5) (width 0.254) (layer B.Cu) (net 3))
 (segment (start 112.618999 106.271001) (end 112.618999 107.881001) (width 0.254) (layer B.Cu) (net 3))
 (segment (start 112.618999 107.881001) (end 108.175 112.325) (width 0.254) (layer B.Cu) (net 3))
 (segment (start 96.25 111.49) (end 104.99 111.49) (width 0.762) (layer F.Cu) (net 3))
 (via (at 104.99 111.49) (size 0.6858) (drill 0.3302) (layers F.Cu B.Cu) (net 3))
 (segment (start 130.075 97.925) (end 132 96) (width 0.254) (layer F.Cu) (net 3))
 (segment (start 132 96) (end 132 94) (width 0.254) (layer F.Cu) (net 3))
 (segment (start 127.95 97.925) (end 130.075 97.925) (width 0.254) (layer F.Cu) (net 3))
 (segment (start 144.38 113.62) (end 148 110) (width 0.762) (layer F.Cu) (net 3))
 (segment (start 148 110) (end 143.381001 105.381001) (width 0.254) (layer B.Cu) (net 3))
 (segment (start 143.381001 105.381001) (end 143.381001 100.377119) (width 0.254) (layer B.Cu) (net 3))
 (segment (start 143.381001 100.377119) (end 141.622881 98.618999) (width 0.254) (layer B.Cu) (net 3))
 (segment (start 135.099882 94) (end 132 94) (width 0.254) (layer B.Cu) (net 3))
 (segment (start 141.622881 98.618999) (end 139.718881 98.618999) (width 0.254) (layer B.Cu) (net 3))
 (segment (start 139.718881 98.618999) (end 135.099882 94) (width 0.254) (layer B.Cu) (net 3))
 (segment (start 140 113.62) (end 144.38 113.62) (width 0.762) (layer F.Cu) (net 3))
 (segment (start 127.95 97.925) (end 113.245 97.925) (width 0.254) (layer B.Cu) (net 3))
 (segment (start 113.245 97.925) (end 112.618999 98.551001) (width 0.254) (layer B.Cu) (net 3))
 (segment (start 112.618999 98.551001) (end 112.618999 106.271001) (width 0.254) (layer B.Cu) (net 3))
 (segment (start 112.618999 106.271001) (end 112.61 106.28) (width 0.254) (layer B.Cu) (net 3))
 (segment (start 111 115.84) (end 109.34 115.84) (width 0.762) (layer F.Cu) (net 3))
 (segment (start 109.34 115.84) (end 107 113.5) (width 0.762) (layer F.Cu) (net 3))
 (segment (start 104.99 111.49) (end 107 113.5) (width 0.762) (layer B.Cu) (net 3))
 (segment (start 120.3 115.205) (end 121.299999 114.205001) (width 0.254) (layer F.Cu) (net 10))
 (segment (start 121.299999 114.205001) (end 125.224999 114.205001) (width 0.254) (layer F.Cu) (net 10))
 (segment (start 125.224999 114.205001) (end 127.175001 112.254999) (width 0.254) (layer F.Cu) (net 10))
 (segment (start 127.175001 112.254999) (end 128.175 111.255) (width 0.254) (layer F.Cu) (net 10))
 (segment (start 103 116.6) (end 107.836872 116.6) (width 0.254) (layer B.Cu) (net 10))
 (segment (start 107.836872 116.6) (end 110.336872 114.1) (width 0.254) (layer B.Cu) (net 10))
 (segment (start 110.336872 114.1) (end 119.195 114.1) (width 0.254) (layer B.Cu) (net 10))
 (segment (start 119.195 114.1) (end 120.3 115.205) (width 0.254) (layer B.Cu) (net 10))
 (segment (start 100.004 116.6) (end 103 116.6) (width 0.254) (layer F.Cu) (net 10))
 (via (at 103 116.6) (size 0.6858) (drill 0.3302) (layers F.Cu B.Cu) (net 10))
 (segment (start 96 116.6) (end 100.004 116.6) (width 0.254) (layer F.Cu) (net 10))
 (segment (start 131.862718 97.94) (end 133.155787 97.94) (width 0.254) (layer B.Cu) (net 11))
 (segment (start 133.155787 97.94) (end 134.57 97.94) (width 0.254) (layer B.Cu) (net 11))
 (segment (start 125.361281 99.163999) (end 127.128283 100.931001) (width 0.254) (layer B.Cu) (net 11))
 (segment (start 121.163999 100.638719) (end 122.638719 99.163999) (width 0.254) (layer B.Cu) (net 11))
 (segment (start 128.871717 100.931001) (end 131.862718 97.94) (width 0.254) (layer B.Cu) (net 11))
 (segment (start 119.69199 111.234128) (end 119.69199 109.12801) (width 0.254) (layer B.Cu) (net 11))
 (segment (start 121.163999 104.343999) (end 121.163999 100.638719) (width 0.254) (layer B.Cu) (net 11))
 (segment (start 127.128283 100.931001) (end 128.871717 100.931001) (width 0.254) (layer B.Cu) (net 11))
 (segment (start 105.023902 115.923902) (end 107.794534 115.923902) (width 0.254) (layer B.Cu) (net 11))
 (segment (start 119.69199 109.12801) (end 122.82 106) (width 0.254) (layer B.Cu) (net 11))
 (segment (start 110.126447 113.591989) (end 117.334129 113.591989) (width 0.254) (layer B.Cu) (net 11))
 (segment (start 117.334129 113.591989) (end 119.69199 111.234128) (width 0.254) (layer B.Cu) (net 11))
 (segment (start 122.82 106) (end 121.163999 104.343999) (width 0.254) (layer B.Cu) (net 11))
 (segment (start 107.794534 115.923902) (end 110.126447 113.591989) (width 0.254) (layer B.Cu) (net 11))
 (segment (start 103.1 114) (end 105.023902 115.923902) (width 0.254) (layer B.Cu) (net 11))
 (segment (start 122.638719 99.163999) (end 125.361281 99.163999) (width 0.254) (layer B.Cu) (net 11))
 (via (at 103.1 114) (size 0.6858) (drill 0.3302) (layers F.Cu B.Cu) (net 11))
 (segment (start 100.004 114) (end 103.1 114) (width 0.254) (layer F.Cu) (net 11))
 (segment (start 96 114) (end 100.004 114) (width 0.254) (layer F.Cu) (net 11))
 (segment (start 116.12 93.97) (end 112.618999 97.471001) (width 0.254) (layer F.Cu) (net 9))
 (segment (start 112.618999 97.471001) (end 112.618999 108.358999) (width 0.254) (layer F.Cu) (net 9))
 (segment (start 112.618999 108.358999) (end 112.63 108.37) (width 0.254) (layer F.Cu) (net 9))
 (segment (start 112.63 108.37) (end 112 109) (width 0.254) (layer F.Cu) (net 9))
 (segment (start 112 109) (end 112 114) (width 0.254) (layer F.Cu) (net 9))
 (segment (start 112 114) (end 116 118) (width 0.254) (layer F.Cu) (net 9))
 (segment (start 127.95 95.925) (end 127.066117 95.925) (width 0.254) (layer F.Cu) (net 9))
 (segment (start 127.066117 95.925) (end 125.141117 94) (width 0.254) (layer F.Cu) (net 9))
 (segment (start 125.141117 94) (end 124 94) (width 0.254) (layer F.Cu) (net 9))
 (segment (start 116 94) (end 124 94) (width 0.254) (layer F.Cu) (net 9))
 (segment (start 116.075 93.925) (end 116 94) (width 0.762) (layer B.Cu) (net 9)))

